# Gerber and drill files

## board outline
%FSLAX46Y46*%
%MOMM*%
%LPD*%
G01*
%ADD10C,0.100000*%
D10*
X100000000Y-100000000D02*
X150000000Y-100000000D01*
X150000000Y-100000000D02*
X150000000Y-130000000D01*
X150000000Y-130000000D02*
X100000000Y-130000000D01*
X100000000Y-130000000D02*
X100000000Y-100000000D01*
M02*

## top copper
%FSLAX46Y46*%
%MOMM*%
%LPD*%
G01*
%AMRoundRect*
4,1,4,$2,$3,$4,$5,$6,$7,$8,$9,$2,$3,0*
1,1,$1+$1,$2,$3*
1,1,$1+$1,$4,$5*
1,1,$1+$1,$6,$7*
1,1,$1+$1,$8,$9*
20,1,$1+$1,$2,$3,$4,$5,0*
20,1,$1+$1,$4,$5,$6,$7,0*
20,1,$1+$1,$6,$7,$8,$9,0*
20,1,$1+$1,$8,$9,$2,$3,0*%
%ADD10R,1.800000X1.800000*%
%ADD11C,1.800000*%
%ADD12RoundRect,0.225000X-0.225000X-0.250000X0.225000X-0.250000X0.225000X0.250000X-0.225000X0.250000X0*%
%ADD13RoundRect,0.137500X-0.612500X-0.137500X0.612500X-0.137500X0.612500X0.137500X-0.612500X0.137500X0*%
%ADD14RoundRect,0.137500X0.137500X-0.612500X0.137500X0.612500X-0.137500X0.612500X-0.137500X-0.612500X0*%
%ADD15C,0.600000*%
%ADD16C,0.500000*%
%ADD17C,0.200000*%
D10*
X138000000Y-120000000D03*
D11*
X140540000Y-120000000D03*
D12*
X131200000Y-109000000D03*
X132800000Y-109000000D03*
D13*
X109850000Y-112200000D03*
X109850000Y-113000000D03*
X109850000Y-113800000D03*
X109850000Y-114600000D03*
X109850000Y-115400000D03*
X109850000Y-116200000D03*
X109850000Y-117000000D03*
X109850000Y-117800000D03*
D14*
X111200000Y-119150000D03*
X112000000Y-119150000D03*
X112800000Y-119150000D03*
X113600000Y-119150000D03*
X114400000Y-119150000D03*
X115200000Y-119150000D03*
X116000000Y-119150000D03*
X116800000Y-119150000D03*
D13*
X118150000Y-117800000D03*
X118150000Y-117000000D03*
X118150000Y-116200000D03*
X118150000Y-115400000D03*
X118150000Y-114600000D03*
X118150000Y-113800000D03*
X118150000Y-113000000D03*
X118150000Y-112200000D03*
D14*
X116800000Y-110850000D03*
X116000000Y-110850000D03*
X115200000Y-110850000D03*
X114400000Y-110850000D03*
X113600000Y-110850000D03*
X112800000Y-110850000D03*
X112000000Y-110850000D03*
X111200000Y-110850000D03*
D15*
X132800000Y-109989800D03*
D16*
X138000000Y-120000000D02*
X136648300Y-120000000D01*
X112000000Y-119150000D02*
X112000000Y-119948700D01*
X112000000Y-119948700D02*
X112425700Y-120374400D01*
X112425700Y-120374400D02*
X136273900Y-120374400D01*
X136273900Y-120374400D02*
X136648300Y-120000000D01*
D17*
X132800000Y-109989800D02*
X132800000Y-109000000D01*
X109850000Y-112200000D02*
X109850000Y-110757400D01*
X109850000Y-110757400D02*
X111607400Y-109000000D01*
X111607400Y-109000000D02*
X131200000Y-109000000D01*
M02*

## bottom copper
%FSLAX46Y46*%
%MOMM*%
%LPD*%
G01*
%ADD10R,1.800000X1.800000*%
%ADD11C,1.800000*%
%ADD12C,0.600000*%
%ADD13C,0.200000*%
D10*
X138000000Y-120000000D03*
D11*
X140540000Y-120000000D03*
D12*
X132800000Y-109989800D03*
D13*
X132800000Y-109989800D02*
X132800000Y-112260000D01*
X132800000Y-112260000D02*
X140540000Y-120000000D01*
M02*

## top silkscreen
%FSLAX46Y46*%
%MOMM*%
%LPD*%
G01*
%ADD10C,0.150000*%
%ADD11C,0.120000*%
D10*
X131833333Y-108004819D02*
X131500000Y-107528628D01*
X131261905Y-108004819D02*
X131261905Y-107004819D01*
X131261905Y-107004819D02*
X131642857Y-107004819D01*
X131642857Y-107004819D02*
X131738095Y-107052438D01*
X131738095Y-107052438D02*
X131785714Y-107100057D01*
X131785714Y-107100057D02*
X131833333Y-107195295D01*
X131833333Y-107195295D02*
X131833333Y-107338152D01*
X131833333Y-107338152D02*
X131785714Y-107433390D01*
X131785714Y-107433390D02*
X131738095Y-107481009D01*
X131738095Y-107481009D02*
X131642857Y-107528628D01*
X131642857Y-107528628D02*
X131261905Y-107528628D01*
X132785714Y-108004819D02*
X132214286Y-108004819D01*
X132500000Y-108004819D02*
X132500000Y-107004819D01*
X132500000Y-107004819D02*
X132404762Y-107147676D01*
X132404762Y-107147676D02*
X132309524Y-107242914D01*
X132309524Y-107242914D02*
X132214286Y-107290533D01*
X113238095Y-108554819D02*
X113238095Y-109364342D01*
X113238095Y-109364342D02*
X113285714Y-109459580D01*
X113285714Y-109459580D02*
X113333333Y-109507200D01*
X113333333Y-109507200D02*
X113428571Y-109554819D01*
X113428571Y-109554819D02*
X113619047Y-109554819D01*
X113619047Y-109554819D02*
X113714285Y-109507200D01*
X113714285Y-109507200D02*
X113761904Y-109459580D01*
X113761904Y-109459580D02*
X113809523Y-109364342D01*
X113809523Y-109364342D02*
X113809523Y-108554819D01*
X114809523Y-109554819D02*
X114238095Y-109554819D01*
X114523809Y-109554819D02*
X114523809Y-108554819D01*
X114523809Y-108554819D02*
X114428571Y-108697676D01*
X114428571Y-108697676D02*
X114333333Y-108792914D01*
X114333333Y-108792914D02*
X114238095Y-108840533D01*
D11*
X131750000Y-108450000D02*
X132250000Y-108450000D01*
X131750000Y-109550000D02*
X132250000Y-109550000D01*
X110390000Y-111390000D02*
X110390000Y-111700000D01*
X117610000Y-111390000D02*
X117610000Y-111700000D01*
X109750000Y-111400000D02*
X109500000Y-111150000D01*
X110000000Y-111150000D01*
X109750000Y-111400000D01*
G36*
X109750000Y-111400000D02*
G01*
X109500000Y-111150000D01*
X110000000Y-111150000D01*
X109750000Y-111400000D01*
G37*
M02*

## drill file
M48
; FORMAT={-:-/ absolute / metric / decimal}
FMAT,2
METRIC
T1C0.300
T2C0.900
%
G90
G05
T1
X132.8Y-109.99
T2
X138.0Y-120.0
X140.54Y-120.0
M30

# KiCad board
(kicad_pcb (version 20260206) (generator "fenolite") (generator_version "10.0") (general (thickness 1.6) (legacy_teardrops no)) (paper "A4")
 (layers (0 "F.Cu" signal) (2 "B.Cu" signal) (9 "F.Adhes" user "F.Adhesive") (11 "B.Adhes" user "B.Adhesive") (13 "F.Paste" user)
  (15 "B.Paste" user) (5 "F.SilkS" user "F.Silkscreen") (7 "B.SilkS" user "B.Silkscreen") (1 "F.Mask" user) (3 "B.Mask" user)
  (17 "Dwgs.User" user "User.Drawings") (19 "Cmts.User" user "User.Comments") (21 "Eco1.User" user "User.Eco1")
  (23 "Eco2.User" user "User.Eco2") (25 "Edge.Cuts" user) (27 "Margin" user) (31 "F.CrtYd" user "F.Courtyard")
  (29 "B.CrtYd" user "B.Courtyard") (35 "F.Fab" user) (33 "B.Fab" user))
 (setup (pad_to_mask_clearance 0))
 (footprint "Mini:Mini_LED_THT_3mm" (layer "B.Cu") (at 138 120)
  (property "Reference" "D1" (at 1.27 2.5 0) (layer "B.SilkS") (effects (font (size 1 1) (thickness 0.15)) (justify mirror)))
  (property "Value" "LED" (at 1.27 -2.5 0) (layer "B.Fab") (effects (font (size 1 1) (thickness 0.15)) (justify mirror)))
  (pad "1" thru_hole rect (at 0 0) (size 1.8 1.8) (drill 0.9) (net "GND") (layers "*.Cu" "*.Mask") (remove_unused_layers no))
  (pad "2" thru_hole circle (at 2.54 0) (size 1.8 1.8) (drill 0.9) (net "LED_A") (layers "*.Cu" "*.Mask") (remove_unused_layers no)))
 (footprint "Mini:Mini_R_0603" (layer "F.Cu") (at 132 109)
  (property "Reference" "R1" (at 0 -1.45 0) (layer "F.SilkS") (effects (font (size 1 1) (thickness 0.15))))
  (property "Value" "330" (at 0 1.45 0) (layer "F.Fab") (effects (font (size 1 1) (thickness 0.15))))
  (fp_line (start -0.25 -0.55) (end 0.25 -0.55) (stroke (width 0.12) (type solid)) (layer "F.SilkS"))
  (fp_line (start -0.25 0.55) (end 0.25 0.55) (stroke (width 0.12) (type solid)) (layer "F.SilkS"))
  (pad "1" smd roundrect (at -0.8 0) (size 0.9 0.95) (layers "F.Cu" "F.Mask" "F.Paste") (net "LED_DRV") (roundrect_rratio 0.25))
  (pad "2" smd roundrect (at 0.8 0) (size 0.9 0.95) (layers "F.Cu" "F.Mask" "F.Paste") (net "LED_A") (roundrect_rratio 0.25)))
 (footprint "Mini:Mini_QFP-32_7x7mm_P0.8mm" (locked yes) (layer "F.Cu") (at 114 115)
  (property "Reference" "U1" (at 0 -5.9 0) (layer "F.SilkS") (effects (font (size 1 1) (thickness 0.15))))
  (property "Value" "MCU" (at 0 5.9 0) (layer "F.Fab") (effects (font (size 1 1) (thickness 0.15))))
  (fp_line (start -3.61 -3.61) (end -3.61 -3.3) (stroke (width 0.12) (type solid)) (layer "F.SilkS"))
  (fp_line (start 3.61 -3.61) (end 3.61 -3.3) (stroke (width 0.12) (type solid)) (layer "F.SilkS"))
  (fp_poly (pts (xy -4.25 -3.6) (xy -4.5 -3.85) (xy -4 -3.85)) (stroke (width 0.12) (type solid)) (fill yes) (layer "F.SilkS"))
  (pad "1" smd roundrect (at -4.15 -2.8) (size 1.5 0.55) (layers "F.Cu" "F.Mask" "F.Paste") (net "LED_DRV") (roundrect_rratio 0.25))
  (pad "2" smd roundrect (at -4.15 -2) (size 1.5 0.55) (layers "F.Cu" "F.Mask" "F.Paste") (roundrect_rratio 0.25))
  (pad "3" smd roundrect (at -4.15 -1.2) (size 1.5 0.55) (layers "F.Cu" "F.Mask" "F.Paste") (roundrect_rratio 0.25))
  (pad "4" smd roundrect (at -4.15 -0.4) (size 1.5 0.55) (layers "F.Cu" "F.Mask" "F.Paste") (roundrect_rratio 0.25))
  (pad "5" smd roundrect (at -4.15 0.4) (size 1.5 0.55) (layers "F.Cu" "F.Mask" "F.Paste") (roundrect_rratio 0.25))
  (pad "6" smd roundrect (at -4.15 1.2) (size 1.5 0.55) (layers "F.Cu" "F.Mask" "F.Paste") (roundrect_rratio 0.25))
  (pad "7" smd roundrect (at -4.15 2) (size 1.5 0.55) (layers "F.Cu" "F.Mask" "F.Paste") (roundrect_rratio 0.25))
  (pad "8" smd roundrect (at -4.15 2.8) (size 1.5 0.55) (layers "F.Cu" "F.Mask" "F.Paste") (roundrect_rratio 0.25))
  (pad "9" smd roundrect (at -2.8 4.15 90) (size 1.5 0.55) (layers "F.Cu" "F.Mask" "F.Paste") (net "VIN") (roundrect_rratio 0.25))
  (pad "10" smd roundrect (at -2 4.15 90) (size 1.5 0.55) (layers "F.Cu" "F.Mask" "F.Paste") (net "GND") (roundrect_rratio 0.25))
  (pad "11" smd roundrect (at -1.2 4.15 90) (size 1.5 0.55) (layers "F.Cu" "F.Mask" "F.Paste") (roundrect_rratio 0.25))
  (pad "12" smd roundrect (at -0.4 4.15 90) (size 1.5 0.55) (layers "F.Cu" "F.Mask" "F.Paste") (roundrect_rratio 0.25))
  (pad "13" smd roundrect (at 0.4 4.15 90) (size 1.5 0.55) (layers "F.Cu" "F.Mask" "F.Paste") (roundrect_rratio 0.25))
  (pad "14" smd roundrect (at 1.2 4.15 90) (size 1.5 0.55) (layers "F.Cu" "F.Mask" "F.Paste") (roundrect_rratio 0.25))
  (pad "15" smd roundrect (at 2 4.15 90) (size 1.5 0.55) (layers "F.Cu" "F.Mask" "F.Paste") (roundrect_rratio 0.25))
  (pad "16" smd roundrect (at 2.8 4.15 90) (size 1.5 0.55) (layers "F.Cu" "F.Mask" "F.Paste") (roundrect_rratio 0.25))
  (pad "17" smd roundrect (at 4.15 2.8) (size 1.5 0.55) (layers "F.Cu" "F.Mask" "F.Paste") (roundrect_rratio 0.25))
  (pad "18" smd roundrect (at 4.15 2) (size 1.5 0.55) (layers "F.Cu" "F.Mask" "F.Paste") (roundrect_rratio 0.25))
  (pad "19" smd roundrect (at 4.15 1.2) (size 1.5 0.55) (layers "F.Cu" "F.Mask" "F.Paste") (roundrect_rratio 0.25))
  (pad "20" smd roundrect (at 4.15 0.4) (size 1.5 0.55) (layers "F.Cu" "F.Mask" "F.Paste") (roundrect_rratio 0.25))
  (pad "21" smd roundrect (at 4.15 -0.4) (size 1.5 0.55) (layers "F.Cu" "F.Mask" "F.Paste") (roundrect_rratio 0.25))
  (pad "22" smd roundrect (at 4.15 -1.2) (size 1.5 0.55) (layers "F.Cu" "F.Mask" "F.Paste") (roundrect_rratio 0.25))
  (pad "23" smd roundrect (at 4.15 -2) (size 1.5 0.55) (layers "F.Cu" "F.Mask" "F.Paste") (roundrect_rratio 0.25))
  (pad "24" smd roundrect (at 4.15 -2.8) (size 1.5 0.55) (layers "F.Cu" "F.Mask" "F.Paste") (roundrect_rratio 0.25))
  (pad "25" smd roundrect (at 2.8 -4.15 90) (size 1.5 0.55) (layers "F.Cu" "F.Mask" "F.Paste") (roundrect_rratio 0.25))
  (pad "26" smd roundrect (at 2 -4.15 90) (size 1.5 0.55) (layers "F.Cu" "F.Mask" "F.Paste") (roundrect_rratio 0.25))
  (pad "27" smd roundrect (at 1.2 -4.15 90) (size 1.5 0.55) (layers "F.Cu" "F.Mask" "F.Paste") (roundrect_rratio 0.25))
  (pad "28" smd roundrect (at 0.4 -4.15 90) (size 1.5 0.55) (layers "F.Cu" "F.Mask" "F.Paste") (roundrect_rratio 0.25))
  (pad "29" smd roundrect (at -0.4 -4.15 90) (size 1.5 0.55) (layers "F.Cu" "F.Mask" "F.Paste") (roundrect_rratio 0.25))
  (pad "30" smd roundrect (at -1.2 -4.15 90) (size 1.5 0.55) (layers "F.Cu" "F.Mask" "F.Paste") (roundrect_rratio 0.25))
  (pad "31" smd roundrect (at -2 -4.15 90) (size 1.5 0.55) (layers "F.Cu" "F.Mask" "F.Paste") (roundrect_rratio 0.25))
  (pad "32" smd roundrect (at -2.8 -4.15 90) (size 1.5 0.55) (layers "F.Cu" "F.Mask" "F.Paste") (roundrect_rratio 0.25)))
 (gr_line (start 100 100) (end 150 100) (stroke (width 0.1) (type solid)) (layer "Edge.Cuts"))
 (gr_line (start 150 100) (end 150 130) (stroke (width 0.1) (type solid)) (layer "Edge.Cuts"))
 (gr_line (start 150 130) (end 100 130) (stroke (width 0.1) (type solid)) (layer "Edge.Cuts"))
 (gr_line (start 100 130) (end 100 100) (stroke (width 0.1) (type solid)) (layer "Edge.Cuts"))
 (segment (start 138 120) (end 136.6483 120) (width 0.5) (layer "F.Cu") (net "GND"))
 (segment (start 112 119.15) (end 112 119.9487) (width 0.5) (layer "F.Cu") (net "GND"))
 (segment (start 112 119.9487) (end 112.4257 120.3744) (width 0.5) (layer "F.Cu") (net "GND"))
 (segment (start 112.4257 120.3744) (end 136.2739 120.3744) (width 0.5) (layer "F.Cu") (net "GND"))
 (segment (start 136.2739 120.3744) (end 136.6483 120) (width 0.5) (layer "F.Cu") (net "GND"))
 (segment (start 132.8 109.9898) (end 132.8 112.26) (width 0.2) (layer "B.Cu") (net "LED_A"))
 (segment (start 132.8 112.26) (end 140.54 120) (width 0.2) (layer "B.Cu") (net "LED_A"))
 (segment (start 132.8 109.9898) (end 132.8 109) (width 0.2) (layer "F.Cu") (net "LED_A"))
 (segment (start 109.85 112.2) (end 109.85 110.7574) (width 0.2) (layer "F.Cu") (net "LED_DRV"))
 (segment (start 109.85 110.7574) (end 111.6074 109) (width 0.2) (layer "F.Cu") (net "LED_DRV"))
 (segment (start 111.6074 109) (end 131.2 109) (width 0.2) (layer "F.Cu") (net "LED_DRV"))
 (via (at 132.8 109.9898) (size 0.6) (drill 0.3) (layers "F.Cu" "B.Cu") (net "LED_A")))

